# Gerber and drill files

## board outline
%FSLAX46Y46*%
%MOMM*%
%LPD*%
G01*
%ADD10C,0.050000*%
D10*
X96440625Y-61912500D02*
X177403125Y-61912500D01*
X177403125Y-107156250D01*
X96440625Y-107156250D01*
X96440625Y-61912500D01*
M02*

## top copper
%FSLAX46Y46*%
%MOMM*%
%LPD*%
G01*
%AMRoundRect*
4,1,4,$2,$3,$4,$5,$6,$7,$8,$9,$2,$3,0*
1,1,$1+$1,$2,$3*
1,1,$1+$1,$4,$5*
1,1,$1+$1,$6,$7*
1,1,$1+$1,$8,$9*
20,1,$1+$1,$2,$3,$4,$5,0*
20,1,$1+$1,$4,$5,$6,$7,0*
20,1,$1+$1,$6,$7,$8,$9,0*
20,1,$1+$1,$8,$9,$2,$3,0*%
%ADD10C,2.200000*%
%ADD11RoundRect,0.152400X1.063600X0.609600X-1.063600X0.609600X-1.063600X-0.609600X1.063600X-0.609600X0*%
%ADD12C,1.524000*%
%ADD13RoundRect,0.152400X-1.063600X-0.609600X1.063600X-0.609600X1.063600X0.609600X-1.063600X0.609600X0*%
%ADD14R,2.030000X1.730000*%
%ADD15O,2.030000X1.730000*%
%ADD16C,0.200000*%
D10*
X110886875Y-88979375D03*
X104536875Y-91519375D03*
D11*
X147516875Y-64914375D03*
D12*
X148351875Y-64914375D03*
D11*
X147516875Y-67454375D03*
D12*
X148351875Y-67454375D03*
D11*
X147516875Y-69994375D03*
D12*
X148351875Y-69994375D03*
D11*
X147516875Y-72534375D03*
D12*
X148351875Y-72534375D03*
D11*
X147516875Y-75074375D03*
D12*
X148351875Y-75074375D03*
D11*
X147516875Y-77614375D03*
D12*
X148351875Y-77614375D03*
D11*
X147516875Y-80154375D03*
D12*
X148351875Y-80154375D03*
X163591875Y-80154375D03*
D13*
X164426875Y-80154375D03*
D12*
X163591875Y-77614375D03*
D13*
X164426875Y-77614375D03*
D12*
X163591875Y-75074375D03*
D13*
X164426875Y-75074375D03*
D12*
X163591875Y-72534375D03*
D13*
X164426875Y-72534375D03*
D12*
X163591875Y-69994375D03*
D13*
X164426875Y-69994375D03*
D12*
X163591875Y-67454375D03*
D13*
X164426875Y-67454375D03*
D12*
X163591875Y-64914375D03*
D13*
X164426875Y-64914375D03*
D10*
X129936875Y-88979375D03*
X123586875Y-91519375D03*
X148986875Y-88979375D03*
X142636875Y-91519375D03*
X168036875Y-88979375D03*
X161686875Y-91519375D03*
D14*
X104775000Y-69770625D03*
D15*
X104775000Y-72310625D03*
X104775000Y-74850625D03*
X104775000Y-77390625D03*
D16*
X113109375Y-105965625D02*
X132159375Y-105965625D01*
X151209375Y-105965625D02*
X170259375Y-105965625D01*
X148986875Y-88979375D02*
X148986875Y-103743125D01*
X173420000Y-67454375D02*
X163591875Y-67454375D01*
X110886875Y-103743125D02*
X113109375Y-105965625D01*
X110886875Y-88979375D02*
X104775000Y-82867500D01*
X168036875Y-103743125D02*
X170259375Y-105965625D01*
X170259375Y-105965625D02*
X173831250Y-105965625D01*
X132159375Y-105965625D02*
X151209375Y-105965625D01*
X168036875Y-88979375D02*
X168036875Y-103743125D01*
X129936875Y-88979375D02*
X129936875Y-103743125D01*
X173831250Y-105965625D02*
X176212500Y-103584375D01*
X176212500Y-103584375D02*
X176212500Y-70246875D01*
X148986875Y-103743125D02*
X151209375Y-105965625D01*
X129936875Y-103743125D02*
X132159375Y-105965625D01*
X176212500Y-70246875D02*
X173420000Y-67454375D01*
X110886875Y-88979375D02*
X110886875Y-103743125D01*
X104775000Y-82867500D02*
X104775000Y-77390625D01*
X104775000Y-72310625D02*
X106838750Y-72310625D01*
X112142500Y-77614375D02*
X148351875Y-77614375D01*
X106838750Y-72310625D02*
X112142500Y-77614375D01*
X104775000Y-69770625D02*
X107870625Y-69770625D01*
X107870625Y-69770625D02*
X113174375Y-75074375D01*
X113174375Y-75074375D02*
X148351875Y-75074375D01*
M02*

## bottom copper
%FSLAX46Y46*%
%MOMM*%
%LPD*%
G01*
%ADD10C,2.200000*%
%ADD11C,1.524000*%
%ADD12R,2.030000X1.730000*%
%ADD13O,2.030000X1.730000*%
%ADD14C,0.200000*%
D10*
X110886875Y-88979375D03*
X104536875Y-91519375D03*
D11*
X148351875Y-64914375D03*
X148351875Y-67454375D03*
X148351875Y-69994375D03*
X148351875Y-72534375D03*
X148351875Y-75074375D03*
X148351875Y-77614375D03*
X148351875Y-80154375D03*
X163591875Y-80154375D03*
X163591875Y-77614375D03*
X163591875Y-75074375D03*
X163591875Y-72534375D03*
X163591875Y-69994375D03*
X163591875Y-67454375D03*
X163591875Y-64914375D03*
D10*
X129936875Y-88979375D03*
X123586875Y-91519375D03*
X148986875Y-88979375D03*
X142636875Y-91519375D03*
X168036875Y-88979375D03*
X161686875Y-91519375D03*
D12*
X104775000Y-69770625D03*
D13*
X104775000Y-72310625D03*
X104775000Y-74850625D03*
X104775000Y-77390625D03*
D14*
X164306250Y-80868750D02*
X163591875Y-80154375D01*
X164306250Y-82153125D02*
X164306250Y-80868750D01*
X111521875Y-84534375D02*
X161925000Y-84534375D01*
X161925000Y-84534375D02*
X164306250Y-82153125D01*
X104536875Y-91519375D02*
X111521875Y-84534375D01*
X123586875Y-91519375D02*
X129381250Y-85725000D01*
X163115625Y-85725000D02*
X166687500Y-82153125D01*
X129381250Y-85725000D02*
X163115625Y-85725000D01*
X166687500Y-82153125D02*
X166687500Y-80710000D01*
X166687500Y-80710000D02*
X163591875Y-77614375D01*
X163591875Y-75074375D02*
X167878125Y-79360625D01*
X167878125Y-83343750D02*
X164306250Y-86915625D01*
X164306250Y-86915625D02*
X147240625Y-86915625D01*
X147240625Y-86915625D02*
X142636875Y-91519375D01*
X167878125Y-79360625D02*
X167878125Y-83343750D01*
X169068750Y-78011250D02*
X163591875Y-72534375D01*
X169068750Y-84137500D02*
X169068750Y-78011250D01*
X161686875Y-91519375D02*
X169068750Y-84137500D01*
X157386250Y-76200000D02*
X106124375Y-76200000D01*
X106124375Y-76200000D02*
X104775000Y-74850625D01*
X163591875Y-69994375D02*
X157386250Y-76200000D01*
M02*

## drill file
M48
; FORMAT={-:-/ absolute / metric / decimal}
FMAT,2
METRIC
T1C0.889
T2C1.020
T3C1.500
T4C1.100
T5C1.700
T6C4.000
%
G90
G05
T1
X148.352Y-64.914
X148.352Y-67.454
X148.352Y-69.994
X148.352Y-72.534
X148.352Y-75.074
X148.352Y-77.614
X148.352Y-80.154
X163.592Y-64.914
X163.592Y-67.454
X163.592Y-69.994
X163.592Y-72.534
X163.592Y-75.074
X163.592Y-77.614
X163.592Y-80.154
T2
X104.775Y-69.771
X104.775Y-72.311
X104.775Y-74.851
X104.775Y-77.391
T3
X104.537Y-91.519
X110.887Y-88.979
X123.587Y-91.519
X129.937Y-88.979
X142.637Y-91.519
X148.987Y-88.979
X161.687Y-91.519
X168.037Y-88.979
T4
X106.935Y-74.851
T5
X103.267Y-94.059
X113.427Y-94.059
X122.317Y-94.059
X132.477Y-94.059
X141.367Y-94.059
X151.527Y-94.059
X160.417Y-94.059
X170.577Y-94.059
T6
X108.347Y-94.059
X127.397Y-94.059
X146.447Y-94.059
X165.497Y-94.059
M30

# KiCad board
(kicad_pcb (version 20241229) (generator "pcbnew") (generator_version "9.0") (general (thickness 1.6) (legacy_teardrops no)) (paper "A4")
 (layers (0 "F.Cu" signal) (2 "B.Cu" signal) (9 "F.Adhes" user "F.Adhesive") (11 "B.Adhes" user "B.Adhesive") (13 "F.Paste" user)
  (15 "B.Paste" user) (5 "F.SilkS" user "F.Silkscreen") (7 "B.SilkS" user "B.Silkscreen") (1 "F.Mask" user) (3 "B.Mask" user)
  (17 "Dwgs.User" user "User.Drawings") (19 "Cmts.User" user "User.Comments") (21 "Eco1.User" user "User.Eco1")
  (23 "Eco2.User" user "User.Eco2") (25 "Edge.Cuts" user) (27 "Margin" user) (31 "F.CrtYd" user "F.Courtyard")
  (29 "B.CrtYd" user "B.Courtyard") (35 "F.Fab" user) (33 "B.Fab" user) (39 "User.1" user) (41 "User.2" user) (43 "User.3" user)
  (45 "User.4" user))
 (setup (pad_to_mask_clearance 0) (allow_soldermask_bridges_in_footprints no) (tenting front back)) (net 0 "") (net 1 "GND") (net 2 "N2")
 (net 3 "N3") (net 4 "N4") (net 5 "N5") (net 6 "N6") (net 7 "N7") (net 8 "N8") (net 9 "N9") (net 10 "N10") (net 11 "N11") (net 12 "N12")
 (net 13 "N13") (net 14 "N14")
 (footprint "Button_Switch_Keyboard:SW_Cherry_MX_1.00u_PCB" (layer "F.Cu") (at 110.886875 88.979375)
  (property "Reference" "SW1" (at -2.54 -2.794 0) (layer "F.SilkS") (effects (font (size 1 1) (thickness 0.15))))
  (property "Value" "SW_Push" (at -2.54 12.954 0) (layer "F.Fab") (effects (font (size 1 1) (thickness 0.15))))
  (pad "" np_thru_hole circle (at -7.62 5.08) (size 1.7 1.7) (drill 1.7) (layers "*.Cu" "*.Mask"))
  (pad "" np_thru_hole circle (at -2.54 5.08) (size 4 4) (drill 4) (layers "*.Cu" "*.Mask"))
  (pad "" np_thru_hole circle (at 2.54 5.08) (size 1.7 1.7) (drill 1.7) (layers "*.Cu" "*.Mask"))
  (pad "1" thru_hole circle (at 0 0) (size 2.2 2.2) (drill 1.5) (layers "*.Cu" "*.Mask") (remove_unused_layers no) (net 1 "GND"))
  (pad "2" thru_hole circle (at -6.35 2.54) (size 2.2 2.2) (drill 1.5) (layers "*.Cu" "*.Mask") (remove_unused_layers no) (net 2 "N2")))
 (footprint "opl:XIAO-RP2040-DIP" (layer "F.Cu") (at 155.971875 72.534375)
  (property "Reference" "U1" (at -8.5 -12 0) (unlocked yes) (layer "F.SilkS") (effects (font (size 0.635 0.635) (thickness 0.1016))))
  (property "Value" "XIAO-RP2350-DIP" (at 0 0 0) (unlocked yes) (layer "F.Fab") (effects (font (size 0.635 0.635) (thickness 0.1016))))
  (pad "1" smd roundrect (at -8.455 -7.62 180) (size 2.432 1.524) (layers "F.Cu" "F.Mask") (roundrect_rratio 0.1) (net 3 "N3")
   (thermal_bridge_angle 45))
  (pad "1" thru_hole circle (at -7.62 -7.62 180) (size 1.524 1.524) (drill 0.889) (layers "*.Cu" "*.Mask") (remove_unused_layers no)
   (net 3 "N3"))
  (pad "2" smd roundrect (at -8.455 -5.08 180) (size 2.432 1.524) (layers "F.Cu" "F.Mask") (roundrect_rratio 0.1) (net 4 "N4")
   (thermal_bridge_angle 45))
  (pad "2" thru_hole circle (at -7.62 -5.08 180) (size 1.524 1.524) (drill 0.889) (layers "*.Cu" "*.Mask") (remove_unused_layers no)
   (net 4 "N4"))
  (pad "3" smd roundrect (at -8.455 -2.54 180) (size 2.432 1.524) (layers "F.Cu" "F.Mask") (roundrect_rratio 0.1) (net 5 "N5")
   (thermal_bridge_angle 45))
  (pad "3" thru_hole circle (at -7.62 -2.54 180) (size 1.524 1.524) (drill 0.889) (layers "*.Cu" "*.Mask") (remove_unused_layers no)
   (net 5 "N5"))
  (pad "4" smd roundrect (at -8.455 0 180) (size 2.432 1.524) (layers "F.Cu" "F.Mask") (roundrect_rratio 0.1) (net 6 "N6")
   (thermal_bridge_angle 45))
  (pad "4" thru_hole circle (at -7.62 0 180) (size 1.524 1.524) (drill 0.889) (layers "*.Cu" "*.Mask") (remove_unused_layers no)
   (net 6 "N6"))
  (pad "5" smd roundrect (at -8.455 2.54 180) (size 2.432 1.524) (layers "F.Cu" "F.Mask") (roundrect_rratio 0.1) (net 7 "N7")
   (thermal_bridge_angle 45))
  (pad "5" thru_hole circle (at -7.62 2.54 180) (size 1.524 1.524) (drill 0.889) (layers "*.Cu" "*.Mask") (remove_unused_layers no)
   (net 7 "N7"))
  (pad "6" smd roundrect (at -8.455 5.08 180) (size 2.432 1.524) (layers "F.Cu" "F.Mask") (roundrect_rratio 0.1) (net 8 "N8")
   (thermal_bridge_angle 45))
  (pad "6" thru_hole circle (at -7.62 5.08 180) (size 1.524 1.524) (drill 0.889) (layers "*.Cu" "*.Mask") (remove_unused_layers no)
   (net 8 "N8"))
  (pad "7" smd roundrect (at -8.455 7.62 180) (size 2.432 1.524) (layers "F.Cu" "F.Mask") (roundrect_rratio 0.1) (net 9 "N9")
   (thermal_bridge_angle 45))
  (pad "7" thru_hole circle (at -7.62 7.62 180) (size 1.524 1.524) (drill 0.889) (layers "*.Cu" "*.Mask") (remove_unused_layers no)
   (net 9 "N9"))
  (pad "8" thru_hole circle (at 7.62 7.62) (size 1.524 1.524) (drill 0.889) (layers "*.Cu" "*.Mask") (remove_unused_layers no) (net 2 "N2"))
  (pad "8" smd roundrect (at 8.455 7.62) (size 2.432 1.524) (layers "F.Cu" "F.Mask") (roundrect_rratio 0.1) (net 2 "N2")
   (thermal_bridge_angle 45))
  (pad "9" thru_hole circle (at 7.62 5.08) (size 1.524 1.524) (drill 0.889) (layers "*.Cu" "*.Mask") (remove_unused_layers no)
   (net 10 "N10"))
  (pad "9" smd roundrect (at 8.455 5.08) (size 2.432 1.524) (layers "F.Cu" "F.Mask") (roundrect_rratio 0.1) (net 10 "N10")
   (thermal_bridge_angle 45))
  (pad "10" thru_hole circle (at 7.62 2.54) (size 1.524 1.524) (drill 0.889) (layers "*.Cu" "*.Mask") (remove_unused_layers no)
   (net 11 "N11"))
  (pad "10" smd roundrect (at 8.455 2.54) (size 2.432 1.524) (layers "F.Cu" "F.Mask") (roundrect_rratio 0.1) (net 11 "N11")
   (thermal_bridge_angle 45))
  (pad "11" thru_hole circle (at 7.62 0) (size 1.524 1.524) (drill 0.889) (layers "*.Cu" "*.Mask") (remove_unused_layers no) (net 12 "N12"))
  (pad "11" smd roundrect (at 8.455 0) (size 2.432 1.524) (layers "F.Cu" "F.Mask") (roundrect_rratio 0.1) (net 12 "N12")
   (thermal_bridge_angle 45))
  (pad "12" thru_hole circle (at 7.62 -2.54) (size 1.524 1.524) (drill 0.889) (layers "*.Cu" "*.Mask") (remove_unused_layers no)
   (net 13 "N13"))
  (pad "12" smd roundrect (at 8.455 -2.54) (size 2.432 1.524) (layers "F.Cu" "F.Mask") (roundrect_rratio 0.1) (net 13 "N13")
   (thermal_bridge_angle 45))
  (pad "13" thru_hole circle (at 7.62 -5.08) (size 1.524 1.524) (drill 0.889) (layers "*.Cu" "*.Mask") (remove_unused_layers no)
   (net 1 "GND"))
  (pad "13" smd roundrect (at 8.455 -5.08) (size 2.432 1.524) (layers "F.Cu" "F.Mask") (roundrect_rratio 0.1) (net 1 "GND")
   (thermal_bridge_angle 45))
  (pad "14" thru_hole circle (at 7.62 -7.62) (size 1.524 1.524) (drill 0.889) (layers "*.Cu" "*.Mask") (remove_unused_layers no)
   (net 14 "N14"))
  (pad "14" smd roundrect (at 8.455 -7.62) (size 2.432 1.524) (layers "F.Cu" "F.Mask") (roundrect_rratio 0.1) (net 14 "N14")
   (thermal_bridge_angle 45)))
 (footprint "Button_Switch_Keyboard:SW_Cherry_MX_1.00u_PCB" (layer "F.Cu") (at 129.936875 88.979375)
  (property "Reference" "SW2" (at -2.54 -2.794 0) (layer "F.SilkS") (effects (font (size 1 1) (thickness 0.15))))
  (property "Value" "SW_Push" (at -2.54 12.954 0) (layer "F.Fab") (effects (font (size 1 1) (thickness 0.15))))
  (pad "" np_thru_hole circle (at -7.62 5.08) (size 1.7 1.7) (drill 1.7) (layers "*.Cu" "*.Mask"))
  (pad "" np_thru_hole circle (at -2.54 5.08) (size 4 4) (drill 4) (layers "*.Cu" "*.Mask"))
  (pad "" np_thru_hole circle (at 2.54 5.08) (size 1.7 1.7) (drill 1.7) (layers "*.Cu" "*.Mask"))
  (pad "1" thru_hole circle (at 0 0) (size 2.2 2.2) (drill 1.5) (layers "*.Cu" "*.Mask") (remove_unused_layers no) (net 1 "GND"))
  (pad "2" thru_hole circle (at -6.35 2.54) (size 2.2 2.2) (drill 1.5) (layers "*.Cu" "*.Mask") (remove_unused_layers no) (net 10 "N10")))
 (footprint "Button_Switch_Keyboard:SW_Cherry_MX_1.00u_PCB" (layer "F.Cu") (at 148.986875 88.979375)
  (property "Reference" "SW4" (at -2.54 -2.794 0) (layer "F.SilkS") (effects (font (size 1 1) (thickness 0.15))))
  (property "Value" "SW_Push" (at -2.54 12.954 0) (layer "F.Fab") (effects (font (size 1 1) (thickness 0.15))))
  (pad "" np_thru_hole circle (at -7.62 5.08) (size 1.7 1.7) (drill 1.7) (layers "*.Cu" "*.Mask"))
  (pad "" np_thru_hole circle (at -2.54 5.08) (size 4 4) (drill 4) (layers "*.Cu" "*.Mask"))
  (pad "" np_thru_hole circle (at 2.54 5.08) (size 1.7 1.7) (drill 1.7) (layers "*.Cu" "*.Mask"))
  (pad "1" thru_hole circle (at 0 0) (size 2.2 2.2) (drill 1.5) (layers "*.Cu" "*.Mask") (remove_unused_layers no) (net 1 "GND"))
  (pad "2" thru_hole circle (at -6.35 2.54) (size 2.2 2.2) (drill 1.5) (layers "*.Cu" "*.Mask") (remove_unused_layers no) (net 11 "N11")))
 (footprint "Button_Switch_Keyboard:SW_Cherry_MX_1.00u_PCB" (layer "F.Cu") (at 168.036875 88.979375)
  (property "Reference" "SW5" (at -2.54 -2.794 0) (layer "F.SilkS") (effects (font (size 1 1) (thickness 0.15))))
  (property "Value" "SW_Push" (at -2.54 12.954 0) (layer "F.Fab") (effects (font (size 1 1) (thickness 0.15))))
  (pad "" np_thru_hole circle (at -7.62 5.08) (size 1.7 1.7) (drill 1.7) (layers "*.Cu" "*.Mask"))
  (pad "" np_thru_hole circle (at -2.54 5.08) (size 4 4) (drill 4) (layers "*.Cu" "*.Mask"))
  (pad "" np_thru_hole circle (at 2.54 5.08) (size 1.7 1.7) (drill 1.7) (layers "*.Cu" "*.Mask"))
  (pad "1" thru_hole circle (at 0 0) (size 2.2 2.2) (drill 1.5) (layers "*.Cu" "*.Mask") (remove_unused_layers no) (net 1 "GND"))
  (pad "2" thru_hole circle (at -6.35 2.54) (size 2.2 2.2) (drill 1.5) (layers "*.Cu" "*.Mask") (remove_unused_layers no) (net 12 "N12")))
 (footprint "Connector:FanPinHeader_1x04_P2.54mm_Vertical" (layer "F.Cu") (at 104.775 69.770625 -90)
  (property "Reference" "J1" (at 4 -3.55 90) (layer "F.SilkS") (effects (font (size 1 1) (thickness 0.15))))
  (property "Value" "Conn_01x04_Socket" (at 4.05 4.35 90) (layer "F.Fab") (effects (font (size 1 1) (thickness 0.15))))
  (pad "" np_thru_hole circle (at 5.08 -2.16) (size 1.1 1.1) (drill 1.1) (layers "*.Cu" "*.Mask"))
  (pad "1" thru_hole rect (at 0 0) (size 2.03 1.73) (drill 1.02) (layers "*.Cu" "*.Mask") (remove_unused_layers no) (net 7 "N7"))
  (pad "2" thru_hole oval (at 2.54 0) (size 2.03 1.73) (drill 1.02) (layers "*.Cu" "*.Mask") (remove_unused_layers no) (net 8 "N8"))
  (pad "3" thru_hole oval (at 5.08 0) (size 2.03 1.73) (drill 1.02) (layers "*.Cu" "*.Mask") (remove_unused_layers no) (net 13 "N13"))
  (pad "4" thru_hole oval (at 7.62 0) (size 2.03 1.73) (drill 1.02) (layers "*.Cu" "*.Mask") (remove_unused_layers no) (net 1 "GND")))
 (gr_rect (start 96.440625 61.9125) (end 177.403125 107.15625) (stroke (width 0.05) (type default)) (fill no) (layer "Edge.Cuts"))
 (segment (start 164.30625 80.86875) (end 163.591875 80.154375) (width 0.2) (layer "B.Cu") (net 2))
 (segment (start 164.30625 82.153125) (end 164.30625 80.86875) (width 0.2) (layer "B.Cu") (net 2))
 (segment (start 111.521875 84.534375) (end 161.925 84.534375) (width 0.2) (layer "B.Cu") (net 2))
 (segment (start 161.925 84.534375) (end 164.30625 82.153125) (width 0.2) (layer "B.Cu") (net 2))
 (segment (start 104.536875 91.519375) (end 111.521875 84.534375) (width 0.2) (layer "B.Cu") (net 2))
 (segment (start 113.109375 105.965625) (end 132.159375 105.965625) (width 0.2) (layer "F.Cu") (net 1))
 (segment (start 151.209375 105.965625) (end 170.259375 105.965625) (width 0.2) (layer "F.Cu") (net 1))
 (segment (start 148.986875 88.979375) (end 148.986875 103.743125) (width 0.2) (layer "F.Cu") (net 1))
 (segment (start 173.42 67.454375) (end 163.591875 67.454375) (width 0.2) (layer "F.Cu") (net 1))
 (segment (start 110.886875 103.743125) (end 113.109375 105.965625) (width 0.2) (layer "F.Cu") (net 1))
 (segment (start 110.886875 88.979375) (end 104.775 82.8675) (width 0.2) (layer "F.Cu") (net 1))
 (segment (start 168.036875 103.743125) (end 170.259375 105.965625) (width 0.2) (layer "F.Cu") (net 1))
 (segment (start 170.259375 105.965625) (end 173.83125 105.965625) (width 0.2) (layer "F.Cu") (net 1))
 (segment (start 132.159375 105.965625) (end 151.209375 105.965625) (width 0.2) (layer "F.Cu") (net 1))
 (segment (start 168.036875 88.979375) (end 168.036875 103.743125) (width 0.2) (layer "F.Cu") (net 1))
 (segment (start 129.936875 88.979375) (end 129.936875 103.743125) (width 0.2) (layer "F.Cu") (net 1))
 (segment (start 173.83125 105.965625) (end 176.2125 103.584375) (width 0.2) (layer "F.Cu") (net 1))
 (segment (start 176.2125 103.584375) (end 176.2125 70.246875) (width 0.2) (layer "F.Cu") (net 1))
 (segment (start 148.986875 103.743125) (end 151.209375 105.965625) (width 0.2) (layer "F.Cu") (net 1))
 (segment (start 129.936875 103.743125) (end 132.159375 105.965625) (width 0.2) (layer "F.Cu") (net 1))
 (segment (start 176.2125 70.246875) (end 173.42 67.454375) (width 0.2) (layer "F.Cu") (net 1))
 (segment (start 110.886875 88.979375) (end 110.886875 103.743125) (width 0.2) (layer "F.Cu") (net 1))
 (segment (start 104.775 82.8675) (end 104.775 77.390625) (width 0.2) (layer "F.Cu") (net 1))
 (segment (start 123.586875 91.519375) (end 129.38125 85.725) (width 0.2) (layer "B.Cu") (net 10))
 (segment (start 163.115625 85.725) (end 166.6875 82.153125) (width 0.2) (layer "B.Cu") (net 10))
 (segment (start 129.38125 85.725) (end 163.115625 85.725) (width 0.2) (layer "B.Cu") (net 10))
 (segment (start 166.6875 82.153125) (end 166.6875 80.71) (width 0.2) (layer "B.Cu") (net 10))
 (segment (start 166.6875 80.71) (end 163.591875 77.614375) (width 0.2) (layer "B.Cu") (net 10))
 (segment (start 163.591875 75.074375) (end 167.878125 79.360625) (width 0.2) (layer "B.Cu") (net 11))
 (segment (start 167.878125 83.34375) (end 164.30625 86.915625) (width 0.2) (layer "B.Cu") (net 11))
 (segment (start 164.30625 86.915625) (end 147.240625 86.915625) (width 0.2) (layer "B.Cu") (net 11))
 (segment (start 147.240625 86.915625) (end 142.636875 91.519375) (width 0.2) (layer "B.Cu") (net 11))
 (segment (start 167.878125 79.360625) (end 167.878125 83.34375) (width 0.2) (layer "B.Cu") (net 11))
 (segment (start 169.06875 78.01125) (end 163.591875 72.534375) (width 0.2) (layer "B.Cu") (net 12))
 (segment (start 169.06875 84.1375) (end 169.06875 78.01125) (width 0.2) (layer "B.Cu") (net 12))
 (segment (start 161.686875 91.519375) (end 169.06875 84.1375) (width 0.2) (layer "B.Cu") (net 12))
 (segment (start 104.775 72.310625) (end 106.83875 72.310625) (width 0.2) (layer "F.Cu") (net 8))
 (segment (start 112.1425 77.614375) (end 148.351875 77.614375) (width 0.2) (layer "F.Cu") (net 8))
 (segment (start 106.83875 72.310625) (end 112.1425 77.614375) (width 0.2) (layer "F.Cu") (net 8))
 (segment (start 104.775 69.770625) (end 107.870625 69.770625) (width 0.2) (layer "F.Cu") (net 7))
 (segment (start 107.870625 69.770625) (end 113.174375 75.074375) (width 0.2) (layer "F.Cu") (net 7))
 (segment (start 113.174375 75.074375) (end 148.351875 75.074375) (width 0.2) (layer "F.Cu") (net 7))
 (segment (start 157.38625 76.2) (end 106.124375 76.2) (width 0.2) (layer "B.Cu") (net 13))
 (segment (start 106.124375 76.2) (end 104.775 74.850625) (width 0.2) (layer "B.Cu") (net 13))
 (segment (start 163.591875 69.994375) (end 157.38625 76.2) (width 0.2) (layer "B.Cu") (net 13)))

